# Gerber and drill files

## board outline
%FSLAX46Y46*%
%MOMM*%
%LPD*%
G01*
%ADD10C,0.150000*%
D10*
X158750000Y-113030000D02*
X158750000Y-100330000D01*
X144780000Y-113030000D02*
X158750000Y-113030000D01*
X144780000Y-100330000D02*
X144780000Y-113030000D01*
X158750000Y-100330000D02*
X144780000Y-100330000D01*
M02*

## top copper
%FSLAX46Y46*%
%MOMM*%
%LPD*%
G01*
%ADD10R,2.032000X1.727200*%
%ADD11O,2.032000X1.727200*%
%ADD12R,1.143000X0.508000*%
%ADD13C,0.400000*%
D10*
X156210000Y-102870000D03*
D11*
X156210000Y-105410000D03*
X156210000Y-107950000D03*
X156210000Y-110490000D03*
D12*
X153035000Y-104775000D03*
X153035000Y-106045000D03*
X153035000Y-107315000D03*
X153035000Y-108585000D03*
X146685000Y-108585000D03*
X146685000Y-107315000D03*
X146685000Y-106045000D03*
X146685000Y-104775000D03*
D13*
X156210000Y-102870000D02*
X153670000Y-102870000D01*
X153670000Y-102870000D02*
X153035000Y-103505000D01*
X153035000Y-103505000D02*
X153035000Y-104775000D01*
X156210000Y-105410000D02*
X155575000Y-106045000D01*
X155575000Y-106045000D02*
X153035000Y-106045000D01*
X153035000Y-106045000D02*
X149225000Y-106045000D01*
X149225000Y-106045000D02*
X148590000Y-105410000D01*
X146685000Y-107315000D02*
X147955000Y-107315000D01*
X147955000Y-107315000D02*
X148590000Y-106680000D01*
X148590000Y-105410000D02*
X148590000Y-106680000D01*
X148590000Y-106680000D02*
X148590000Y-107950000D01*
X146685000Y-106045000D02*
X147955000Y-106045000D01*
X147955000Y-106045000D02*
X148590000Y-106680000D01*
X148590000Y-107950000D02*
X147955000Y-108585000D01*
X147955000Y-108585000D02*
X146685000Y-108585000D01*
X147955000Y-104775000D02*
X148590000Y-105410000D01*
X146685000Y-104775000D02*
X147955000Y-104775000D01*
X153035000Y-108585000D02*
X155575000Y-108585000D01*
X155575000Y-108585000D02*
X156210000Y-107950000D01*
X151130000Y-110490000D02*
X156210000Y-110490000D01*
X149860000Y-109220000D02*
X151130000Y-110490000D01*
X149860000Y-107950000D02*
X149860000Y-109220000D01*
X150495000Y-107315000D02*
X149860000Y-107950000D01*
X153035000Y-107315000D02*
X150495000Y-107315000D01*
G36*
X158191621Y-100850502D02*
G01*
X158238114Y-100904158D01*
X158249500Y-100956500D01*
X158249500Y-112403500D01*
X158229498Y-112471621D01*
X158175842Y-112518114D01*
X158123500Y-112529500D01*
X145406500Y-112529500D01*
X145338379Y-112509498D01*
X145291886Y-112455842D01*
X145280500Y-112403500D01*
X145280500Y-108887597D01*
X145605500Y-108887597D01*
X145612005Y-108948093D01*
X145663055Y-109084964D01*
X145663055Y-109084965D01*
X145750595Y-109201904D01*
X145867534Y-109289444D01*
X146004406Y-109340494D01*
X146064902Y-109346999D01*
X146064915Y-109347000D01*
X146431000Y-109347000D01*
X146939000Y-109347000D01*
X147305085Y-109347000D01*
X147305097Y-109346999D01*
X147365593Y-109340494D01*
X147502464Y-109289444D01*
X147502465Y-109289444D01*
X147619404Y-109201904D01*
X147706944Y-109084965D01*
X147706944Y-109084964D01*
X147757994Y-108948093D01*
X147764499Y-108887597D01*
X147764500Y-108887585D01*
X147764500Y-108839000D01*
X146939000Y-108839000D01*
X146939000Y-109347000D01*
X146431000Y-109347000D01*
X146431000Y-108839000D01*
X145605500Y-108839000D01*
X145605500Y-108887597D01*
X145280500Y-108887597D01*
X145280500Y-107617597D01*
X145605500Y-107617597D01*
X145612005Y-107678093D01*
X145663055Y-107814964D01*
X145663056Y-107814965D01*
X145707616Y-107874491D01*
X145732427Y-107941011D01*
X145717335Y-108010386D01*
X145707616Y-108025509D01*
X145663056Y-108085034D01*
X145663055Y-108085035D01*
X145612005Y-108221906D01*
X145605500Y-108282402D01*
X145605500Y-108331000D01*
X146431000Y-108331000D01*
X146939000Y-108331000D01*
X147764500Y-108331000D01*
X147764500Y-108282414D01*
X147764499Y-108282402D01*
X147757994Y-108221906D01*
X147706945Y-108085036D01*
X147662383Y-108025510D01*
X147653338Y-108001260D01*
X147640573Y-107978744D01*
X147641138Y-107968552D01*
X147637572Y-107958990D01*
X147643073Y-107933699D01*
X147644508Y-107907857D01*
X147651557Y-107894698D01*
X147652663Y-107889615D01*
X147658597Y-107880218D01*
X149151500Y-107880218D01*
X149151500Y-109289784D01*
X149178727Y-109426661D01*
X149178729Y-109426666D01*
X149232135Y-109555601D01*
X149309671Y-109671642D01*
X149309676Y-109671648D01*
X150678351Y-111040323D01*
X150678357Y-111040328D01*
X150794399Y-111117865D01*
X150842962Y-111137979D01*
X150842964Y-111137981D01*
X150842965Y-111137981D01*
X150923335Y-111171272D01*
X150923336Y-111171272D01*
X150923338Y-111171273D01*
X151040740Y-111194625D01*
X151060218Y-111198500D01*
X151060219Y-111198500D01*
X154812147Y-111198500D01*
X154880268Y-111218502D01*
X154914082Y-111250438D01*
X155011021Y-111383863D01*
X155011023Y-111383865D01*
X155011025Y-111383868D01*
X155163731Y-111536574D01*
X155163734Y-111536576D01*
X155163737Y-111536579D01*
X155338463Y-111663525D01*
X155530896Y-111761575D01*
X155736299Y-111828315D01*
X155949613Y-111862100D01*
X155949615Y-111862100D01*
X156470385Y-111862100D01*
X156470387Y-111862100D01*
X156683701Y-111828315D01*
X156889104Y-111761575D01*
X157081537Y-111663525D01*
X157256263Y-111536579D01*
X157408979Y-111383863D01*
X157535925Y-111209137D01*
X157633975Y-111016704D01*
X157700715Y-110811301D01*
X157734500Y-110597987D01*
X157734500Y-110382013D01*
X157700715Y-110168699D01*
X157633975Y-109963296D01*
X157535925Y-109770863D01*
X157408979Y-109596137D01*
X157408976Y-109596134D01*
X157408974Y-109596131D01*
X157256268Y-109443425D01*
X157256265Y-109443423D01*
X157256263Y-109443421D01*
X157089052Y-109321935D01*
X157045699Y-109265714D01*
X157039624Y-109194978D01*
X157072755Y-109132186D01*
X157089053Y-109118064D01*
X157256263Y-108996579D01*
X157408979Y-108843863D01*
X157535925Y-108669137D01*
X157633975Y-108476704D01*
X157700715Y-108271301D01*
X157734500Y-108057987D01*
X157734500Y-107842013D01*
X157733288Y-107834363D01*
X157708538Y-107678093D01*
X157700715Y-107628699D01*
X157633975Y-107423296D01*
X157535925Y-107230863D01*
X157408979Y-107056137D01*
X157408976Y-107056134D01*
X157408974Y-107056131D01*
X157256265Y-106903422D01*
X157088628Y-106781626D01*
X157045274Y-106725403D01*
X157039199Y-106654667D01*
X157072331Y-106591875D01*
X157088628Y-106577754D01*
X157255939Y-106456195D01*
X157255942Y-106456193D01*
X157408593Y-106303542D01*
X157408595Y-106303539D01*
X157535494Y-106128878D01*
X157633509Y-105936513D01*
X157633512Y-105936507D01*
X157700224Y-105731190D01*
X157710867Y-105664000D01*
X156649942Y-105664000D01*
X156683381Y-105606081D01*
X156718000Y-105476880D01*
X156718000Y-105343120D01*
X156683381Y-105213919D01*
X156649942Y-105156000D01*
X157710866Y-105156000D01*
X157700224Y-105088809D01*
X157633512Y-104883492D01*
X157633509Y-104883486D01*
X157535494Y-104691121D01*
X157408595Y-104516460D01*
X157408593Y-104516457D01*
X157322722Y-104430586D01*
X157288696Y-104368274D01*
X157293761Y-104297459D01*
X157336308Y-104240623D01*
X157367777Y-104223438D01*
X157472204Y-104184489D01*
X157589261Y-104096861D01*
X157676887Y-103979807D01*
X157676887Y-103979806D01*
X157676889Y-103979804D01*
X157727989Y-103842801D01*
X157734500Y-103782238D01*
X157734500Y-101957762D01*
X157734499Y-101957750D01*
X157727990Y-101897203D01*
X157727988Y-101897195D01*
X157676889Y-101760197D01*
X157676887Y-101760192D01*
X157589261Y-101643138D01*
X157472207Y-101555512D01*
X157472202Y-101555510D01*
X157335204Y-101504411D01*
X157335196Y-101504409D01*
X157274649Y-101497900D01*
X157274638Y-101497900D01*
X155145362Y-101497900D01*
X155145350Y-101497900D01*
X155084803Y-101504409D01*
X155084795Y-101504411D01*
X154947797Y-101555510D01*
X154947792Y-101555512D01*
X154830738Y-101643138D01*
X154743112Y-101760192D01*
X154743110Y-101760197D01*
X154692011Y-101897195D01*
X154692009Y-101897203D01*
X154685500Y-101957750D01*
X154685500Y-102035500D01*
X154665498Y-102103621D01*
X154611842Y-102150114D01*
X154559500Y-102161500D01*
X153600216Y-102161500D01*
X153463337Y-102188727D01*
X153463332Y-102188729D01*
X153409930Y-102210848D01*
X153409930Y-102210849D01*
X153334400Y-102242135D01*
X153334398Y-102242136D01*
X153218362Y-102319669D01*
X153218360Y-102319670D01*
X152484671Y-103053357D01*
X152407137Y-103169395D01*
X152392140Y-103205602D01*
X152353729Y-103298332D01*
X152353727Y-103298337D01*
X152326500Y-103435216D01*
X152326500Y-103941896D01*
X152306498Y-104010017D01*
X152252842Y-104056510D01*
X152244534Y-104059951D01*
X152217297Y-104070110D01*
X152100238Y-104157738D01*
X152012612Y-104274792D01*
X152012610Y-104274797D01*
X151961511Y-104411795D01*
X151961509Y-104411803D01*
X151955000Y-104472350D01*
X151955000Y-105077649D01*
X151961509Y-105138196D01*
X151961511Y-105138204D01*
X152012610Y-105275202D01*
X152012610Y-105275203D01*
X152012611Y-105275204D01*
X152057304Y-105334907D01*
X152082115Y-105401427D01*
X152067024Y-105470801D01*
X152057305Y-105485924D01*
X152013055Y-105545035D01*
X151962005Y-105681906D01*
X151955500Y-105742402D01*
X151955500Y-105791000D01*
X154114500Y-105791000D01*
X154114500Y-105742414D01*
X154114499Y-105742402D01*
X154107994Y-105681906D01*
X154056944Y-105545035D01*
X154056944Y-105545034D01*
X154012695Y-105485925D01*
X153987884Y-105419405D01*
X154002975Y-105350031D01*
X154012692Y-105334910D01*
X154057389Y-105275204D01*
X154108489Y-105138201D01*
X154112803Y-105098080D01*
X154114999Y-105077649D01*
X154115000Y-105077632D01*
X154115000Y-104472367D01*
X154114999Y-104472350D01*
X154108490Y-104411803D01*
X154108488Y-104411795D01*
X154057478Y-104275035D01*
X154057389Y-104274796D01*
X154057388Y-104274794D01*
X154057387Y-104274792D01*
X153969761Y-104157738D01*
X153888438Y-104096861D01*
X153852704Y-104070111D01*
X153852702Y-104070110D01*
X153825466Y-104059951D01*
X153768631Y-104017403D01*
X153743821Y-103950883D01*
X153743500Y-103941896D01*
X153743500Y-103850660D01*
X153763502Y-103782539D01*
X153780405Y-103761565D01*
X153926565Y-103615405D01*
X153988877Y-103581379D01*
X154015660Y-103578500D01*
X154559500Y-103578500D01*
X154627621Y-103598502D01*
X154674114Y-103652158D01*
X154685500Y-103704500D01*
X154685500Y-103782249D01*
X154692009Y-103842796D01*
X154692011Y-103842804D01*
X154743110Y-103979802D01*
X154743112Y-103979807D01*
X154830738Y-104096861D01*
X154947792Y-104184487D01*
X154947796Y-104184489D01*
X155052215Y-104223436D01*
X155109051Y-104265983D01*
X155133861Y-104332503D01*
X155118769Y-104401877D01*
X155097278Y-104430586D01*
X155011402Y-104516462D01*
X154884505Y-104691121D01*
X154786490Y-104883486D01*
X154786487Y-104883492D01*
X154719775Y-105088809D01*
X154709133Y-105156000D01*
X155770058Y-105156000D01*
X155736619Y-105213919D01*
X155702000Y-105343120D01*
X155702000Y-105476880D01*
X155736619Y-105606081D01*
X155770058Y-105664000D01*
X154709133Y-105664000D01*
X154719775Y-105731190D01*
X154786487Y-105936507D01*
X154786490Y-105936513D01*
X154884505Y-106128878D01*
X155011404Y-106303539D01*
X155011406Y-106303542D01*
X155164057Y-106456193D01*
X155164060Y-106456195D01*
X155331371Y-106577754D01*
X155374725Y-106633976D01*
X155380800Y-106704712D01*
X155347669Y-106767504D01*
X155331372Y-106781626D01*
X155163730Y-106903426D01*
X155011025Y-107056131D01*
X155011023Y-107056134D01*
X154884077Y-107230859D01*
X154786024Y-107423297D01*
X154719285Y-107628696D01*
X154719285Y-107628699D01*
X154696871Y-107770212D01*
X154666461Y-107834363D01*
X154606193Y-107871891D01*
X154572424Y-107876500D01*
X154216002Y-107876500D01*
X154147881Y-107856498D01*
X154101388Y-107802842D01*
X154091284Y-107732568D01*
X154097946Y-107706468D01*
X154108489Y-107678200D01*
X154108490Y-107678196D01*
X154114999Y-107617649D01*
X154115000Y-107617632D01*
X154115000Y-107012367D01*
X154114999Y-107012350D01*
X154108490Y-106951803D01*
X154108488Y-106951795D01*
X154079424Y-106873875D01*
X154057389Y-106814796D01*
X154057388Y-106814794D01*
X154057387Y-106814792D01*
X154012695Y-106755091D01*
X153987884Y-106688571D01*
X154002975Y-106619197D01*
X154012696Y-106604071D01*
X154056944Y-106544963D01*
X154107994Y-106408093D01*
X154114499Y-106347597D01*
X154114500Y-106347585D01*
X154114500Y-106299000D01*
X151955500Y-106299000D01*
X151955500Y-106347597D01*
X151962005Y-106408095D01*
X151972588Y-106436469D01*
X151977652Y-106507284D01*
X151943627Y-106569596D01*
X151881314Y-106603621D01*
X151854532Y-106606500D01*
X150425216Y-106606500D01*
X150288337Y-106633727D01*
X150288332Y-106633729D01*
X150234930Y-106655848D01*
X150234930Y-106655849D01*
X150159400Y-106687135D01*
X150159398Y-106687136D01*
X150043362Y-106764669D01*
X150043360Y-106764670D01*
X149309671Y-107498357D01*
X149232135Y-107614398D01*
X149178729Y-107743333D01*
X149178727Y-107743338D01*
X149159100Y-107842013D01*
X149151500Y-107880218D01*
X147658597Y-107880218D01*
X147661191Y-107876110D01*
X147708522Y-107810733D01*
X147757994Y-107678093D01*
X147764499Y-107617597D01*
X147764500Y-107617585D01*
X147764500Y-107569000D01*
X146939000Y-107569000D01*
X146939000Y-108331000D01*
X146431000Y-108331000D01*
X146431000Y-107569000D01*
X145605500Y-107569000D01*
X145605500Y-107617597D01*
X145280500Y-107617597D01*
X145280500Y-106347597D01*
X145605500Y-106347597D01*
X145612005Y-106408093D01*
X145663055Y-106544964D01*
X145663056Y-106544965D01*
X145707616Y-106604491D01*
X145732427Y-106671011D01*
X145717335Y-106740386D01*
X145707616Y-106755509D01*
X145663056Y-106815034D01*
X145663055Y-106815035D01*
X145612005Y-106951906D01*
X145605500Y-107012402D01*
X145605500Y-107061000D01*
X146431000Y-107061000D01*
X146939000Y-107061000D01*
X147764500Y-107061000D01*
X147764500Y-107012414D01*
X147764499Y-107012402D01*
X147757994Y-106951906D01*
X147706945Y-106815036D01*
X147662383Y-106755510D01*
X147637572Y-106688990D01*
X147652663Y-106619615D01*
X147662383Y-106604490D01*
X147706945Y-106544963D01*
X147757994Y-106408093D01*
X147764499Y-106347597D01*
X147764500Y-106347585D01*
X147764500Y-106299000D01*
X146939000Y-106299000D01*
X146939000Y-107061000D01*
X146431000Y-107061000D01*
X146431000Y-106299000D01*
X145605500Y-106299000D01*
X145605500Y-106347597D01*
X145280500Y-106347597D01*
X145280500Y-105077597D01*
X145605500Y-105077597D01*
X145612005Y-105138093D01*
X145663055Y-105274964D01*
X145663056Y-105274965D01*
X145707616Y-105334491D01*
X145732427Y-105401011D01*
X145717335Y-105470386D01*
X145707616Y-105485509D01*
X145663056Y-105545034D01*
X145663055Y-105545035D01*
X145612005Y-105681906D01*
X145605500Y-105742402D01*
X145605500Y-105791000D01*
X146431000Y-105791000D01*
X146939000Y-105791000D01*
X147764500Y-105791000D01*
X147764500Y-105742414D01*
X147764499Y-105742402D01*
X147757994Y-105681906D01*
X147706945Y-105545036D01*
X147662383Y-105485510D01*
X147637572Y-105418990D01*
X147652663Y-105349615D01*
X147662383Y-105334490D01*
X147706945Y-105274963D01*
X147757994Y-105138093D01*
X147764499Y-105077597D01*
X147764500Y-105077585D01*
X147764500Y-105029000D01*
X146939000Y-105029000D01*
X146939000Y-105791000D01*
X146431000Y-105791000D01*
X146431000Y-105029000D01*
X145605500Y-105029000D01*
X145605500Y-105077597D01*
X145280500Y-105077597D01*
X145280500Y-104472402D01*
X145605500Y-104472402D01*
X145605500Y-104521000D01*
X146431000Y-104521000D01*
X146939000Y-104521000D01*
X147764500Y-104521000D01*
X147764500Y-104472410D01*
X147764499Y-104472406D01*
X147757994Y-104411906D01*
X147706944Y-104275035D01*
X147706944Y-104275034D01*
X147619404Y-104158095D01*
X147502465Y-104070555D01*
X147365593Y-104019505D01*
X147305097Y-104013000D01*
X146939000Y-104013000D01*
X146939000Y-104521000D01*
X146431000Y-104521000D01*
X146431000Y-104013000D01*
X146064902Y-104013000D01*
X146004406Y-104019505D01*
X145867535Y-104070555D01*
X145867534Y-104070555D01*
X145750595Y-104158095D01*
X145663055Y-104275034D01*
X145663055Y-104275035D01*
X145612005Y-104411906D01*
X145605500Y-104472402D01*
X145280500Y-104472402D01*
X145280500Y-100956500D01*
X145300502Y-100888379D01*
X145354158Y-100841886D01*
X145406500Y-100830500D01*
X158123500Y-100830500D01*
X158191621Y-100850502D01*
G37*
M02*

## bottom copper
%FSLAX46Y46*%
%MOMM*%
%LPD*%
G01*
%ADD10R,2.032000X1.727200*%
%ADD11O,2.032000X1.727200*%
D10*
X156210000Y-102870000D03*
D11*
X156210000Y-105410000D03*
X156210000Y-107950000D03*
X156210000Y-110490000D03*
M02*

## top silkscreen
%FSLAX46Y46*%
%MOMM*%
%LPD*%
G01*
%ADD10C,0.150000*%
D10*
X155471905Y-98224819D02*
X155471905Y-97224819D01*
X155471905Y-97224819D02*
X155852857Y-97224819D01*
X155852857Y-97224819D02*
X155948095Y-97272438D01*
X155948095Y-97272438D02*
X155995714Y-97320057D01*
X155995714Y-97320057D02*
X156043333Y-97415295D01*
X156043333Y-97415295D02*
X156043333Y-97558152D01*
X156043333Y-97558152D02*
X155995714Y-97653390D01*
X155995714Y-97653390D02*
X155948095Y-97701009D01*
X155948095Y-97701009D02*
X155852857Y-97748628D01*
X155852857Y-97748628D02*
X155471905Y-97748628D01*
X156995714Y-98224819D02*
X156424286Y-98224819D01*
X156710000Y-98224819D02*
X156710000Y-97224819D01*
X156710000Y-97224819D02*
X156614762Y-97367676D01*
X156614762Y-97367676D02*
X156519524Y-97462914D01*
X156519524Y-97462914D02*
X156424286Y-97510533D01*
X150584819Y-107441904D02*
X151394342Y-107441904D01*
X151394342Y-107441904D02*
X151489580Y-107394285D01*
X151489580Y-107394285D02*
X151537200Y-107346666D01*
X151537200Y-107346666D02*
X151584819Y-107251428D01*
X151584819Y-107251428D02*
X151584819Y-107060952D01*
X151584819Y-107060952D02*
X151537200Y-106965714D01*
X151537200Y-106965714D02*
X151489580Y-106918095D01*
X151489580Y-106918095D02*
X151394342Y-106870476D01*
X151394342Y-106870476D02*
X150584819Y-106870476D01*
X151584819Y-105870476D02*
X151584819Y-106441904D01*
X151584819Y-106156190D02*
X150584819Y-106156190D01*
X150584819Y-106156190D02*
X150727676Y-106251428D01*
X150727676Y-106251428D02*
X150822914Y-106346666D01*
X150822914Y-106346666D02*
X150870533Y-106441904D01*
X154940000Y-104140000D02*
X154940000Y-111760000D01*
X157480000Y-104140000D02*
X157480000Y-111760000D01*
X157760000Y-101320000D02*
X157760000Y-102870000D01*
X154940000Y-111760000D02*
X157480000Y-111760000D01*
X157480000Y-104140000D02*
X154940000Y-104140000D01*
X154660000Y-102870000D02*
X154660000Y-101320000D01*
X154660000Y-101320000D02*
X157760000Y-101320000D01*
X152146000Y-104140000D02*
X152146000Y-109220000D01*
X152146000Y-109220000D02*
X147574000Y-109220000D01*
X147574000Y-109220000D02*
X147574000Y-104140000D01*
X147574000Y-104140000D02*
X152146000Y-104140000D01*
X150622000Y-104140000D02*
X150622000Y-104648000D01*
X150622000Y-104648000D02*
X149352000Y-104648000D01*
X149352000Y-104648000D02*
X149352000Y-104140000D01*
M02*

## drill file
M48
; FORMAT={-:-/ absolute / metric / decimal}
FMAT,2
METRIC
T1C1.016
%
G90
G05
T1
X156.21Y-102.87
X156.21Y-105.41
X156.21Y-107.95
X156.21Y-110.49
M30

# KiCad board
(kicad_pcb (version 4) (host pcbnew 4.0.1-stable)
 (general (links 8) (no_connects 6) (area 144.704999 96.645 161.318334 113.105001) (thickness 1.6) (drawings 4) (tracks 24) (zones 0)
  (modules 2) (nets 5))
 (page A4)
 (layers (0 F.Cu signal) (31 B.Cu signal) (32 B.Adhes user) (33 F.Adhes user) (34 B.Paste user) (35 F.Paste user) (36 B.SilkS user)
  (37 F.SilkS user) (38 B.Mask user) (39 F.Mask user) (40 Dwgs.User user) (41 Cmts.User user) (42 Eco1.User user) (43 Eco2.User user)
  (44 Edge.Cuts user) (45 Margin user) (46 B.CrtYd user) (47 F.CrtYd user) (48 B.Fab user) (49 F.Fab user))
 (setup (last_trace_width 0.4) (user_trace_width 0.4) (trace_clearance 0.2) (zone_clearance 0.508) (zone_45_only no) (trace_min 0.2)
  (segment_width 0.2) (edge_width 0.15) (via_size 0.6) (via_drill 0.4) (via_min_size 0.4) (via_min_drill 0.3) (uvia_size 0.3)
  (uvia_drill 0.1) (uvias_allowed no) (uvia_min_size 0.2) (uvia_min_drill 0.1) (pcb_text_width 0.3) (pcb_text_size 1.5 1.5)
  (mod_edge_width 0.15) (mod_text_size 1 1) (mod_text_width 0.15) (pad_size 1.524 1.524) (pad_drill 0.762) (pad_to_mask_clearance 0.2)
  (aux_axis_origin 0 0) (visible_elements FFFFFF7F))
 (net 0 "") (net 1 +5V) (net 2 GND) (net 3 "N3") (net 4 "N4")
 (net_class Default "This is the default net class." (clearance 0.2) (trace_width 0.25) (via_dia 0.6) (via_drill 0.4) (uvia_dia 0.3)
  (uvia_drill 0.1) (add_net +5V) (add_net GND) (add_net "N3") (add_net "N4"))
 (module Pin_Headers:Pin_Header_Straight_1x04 (layer F.Cu) (at 156.21 102.87)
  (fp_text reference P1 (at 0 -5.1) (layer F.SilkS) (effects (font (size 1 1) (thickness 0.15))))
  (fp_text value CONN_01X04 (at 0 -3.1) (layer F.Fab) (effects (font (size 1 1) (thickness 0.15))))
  (fp_line (start -1.27 1.27) (end -1.27 8.89) (layer F.SilkS) (width 0.15))
  (fp_line (start 1.27 1.27) (end 1.27 8.89) (layer F.SilkS) (width 0.15))
  (fp_line (start 1.55 -1.55) (end 1.55 0) (layer F.SilkS) (width 0.15))
  (fp_line (start -1.27 8.89) (end 1.27 8.89) (layer F.SilkS) (width 0.15))
  (fp_line (start 1.27 1.27) (end -1.27 1.27) (layer F.SilkS) (width 0.15))
  (fp_line (start -1.55 0) (end -1.55 -1.55) (layer F.SilkS) (width 0.15))
  (fp_line (start -1.55 -1.55) (end 1.55 -1.55) (layer F.SilkS) (width 0.15))
  (pad 1 thru_hole rect (at 0 0) (size 2.032 1.7272) (drill 1.016) (layers *.Cu *.Mask) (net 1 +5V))
  (pad 2 thru_hole oval (at 0 2.54) (size 2.032 1.7272) (drill 1.016) (layers *.Cu *.Mask) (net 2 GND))
  (pad 3 thru_hole oval (at 0 5.08) (size 2.032 1.7272) (drill 1.016) (layers *.Cu *.Mask) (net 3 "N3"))
  (pad 4 thru_hole oval (at 0 7.62) (size 2.032 1.7272) (drill 1.016) (layers *.Cu *.Mask) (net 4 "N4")))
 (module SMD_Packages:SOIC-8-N (layer F.Cu) (at 149.86 106.68 270)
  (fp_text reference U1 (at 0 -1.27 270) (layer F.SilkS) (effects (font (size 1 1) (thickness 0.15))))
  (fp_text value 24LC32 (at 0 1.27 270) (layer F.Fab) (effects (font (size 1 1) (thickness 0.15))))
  (fp_line (start -2.54 -2.286) (end 2.54 -2.286) (layer F.SilkS) (width 0.15))
  (fp_line (start 2.54 -2.286) (end 2.54 2.286) (layer F.SilkS) (width 0.15))
  (fp_line (start 2.54 2.286) (end -2.54 2.286) (layer F.SilkS) (width 0.15))
  (fp_line (start -2.54 2.286) (end -2.54 -2.286) (layer F.SilkS) (width 0.15))
  (fp_line (start -2.54 -0.762) (end -2.032 -0.762) (layer F.SilkS) (width 0.15))
  (fp_line (start -2.032 -0.762) (end -2.032 0.508) (layer F.SilkS) (width 0.15))
  (fp_line (start -2.032 0.508) (end -2.54 0.508) (layer F.SilkS) (width 0.15))
  (pad 8 smd rect (at -1.905 -3.175 270) (size 0.508 1.143) (layers F.Cu F.Paste F.Mask) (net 1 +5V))
  (pad 7 smd rect (at -0.635 -3.175 270) (size 0.508 1.143) (layers F.Cu F.Paste F.Mask) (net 2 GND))
  (pad 6 smd rect (at 0.635 -3.175 270) (size 0.508 1.143) (layers F.Cu F.Paste F.Mask) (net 4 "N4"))
  (pad 5 smd rect (at 1.905 -3.175 270) (size 0.508 1.143) (layers F.Cu F.Paste F.Mask) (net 3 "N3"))
  (pad 4 smd rect (at 1.905 3.175 270) (size 0.508 1.143) (layers F.Cu F.Paste F.Mask) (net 2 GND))
  (pad 3 smd rect (at 0.635 3.175 270) (size 0.508 1.143) (layers F.Cu F.Paste F.Mask) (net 2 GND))
  (pad 2 smd rect (at -0.635 3.175 270) (size 0.508 1.143) (layers F.Cu F.Paste F.Mask) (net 2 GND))
  (pad 1 smd rect (at -1.905 3.175 270) (size 0.508 1.143) (layers F.Cu F.Paste F.Mask) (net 2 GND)))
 (gr_line (start 158.75 113.03) (end 158.75 100.33) (layer Edge.Cuts) (width 0.15))
 (gr_line (start 144.78 113.03) (end 158.75 113.03) (layer Edge.Cuts) (width 0.15))
 (gr_line (start 144.78 100.33) (end 144.78 113.03) (layer Edge.Cuts) (width 0.15))
 (gr_line (start 158.75 100.33) (end 144.78 100.33) (layer Edge.Cuts) (width 0.15))
 (segment (start 156.21 102.87) (end 153.67 102.87) (width 0.4) (layer F.Cu) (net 1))
 (segment (start 153.67 102.87) (end 153.035 103.505) (width 0.4) (layer F.Cu) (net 1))
 (segment (start 153.035 103.505) (end 153.035 104.775) (width 0.4) (layer F.Cu) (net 1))
 (segment (start 156.21 105.41) (end 155.575 106.045) (width 0.4) (layer F.Cu) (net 2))
 (segment (start 155.575 106.045) (end 153.035 106.045) (width 0.4) (layer F.Cu) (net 2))
 (segment (start 153.035 106.045) (end 149.225 106.045) (width 0.4) (layer F.Cu) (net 2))
 (segment (start 149.225 106.045) (end 148.59 105.41) (width 0.4) (layer F.Cu) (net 2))
 (segment (start 146.685 107.315) (end 147.955 107.315) (width 0.4) (layer F.Cu) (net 2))
 (segment (start 147.955 107.315) (end 148.59 106.68) (width 0.4) (layer F.Cu) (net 2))
 (segment (start 148.59 105.41) (end 148.59 106.68) (width 0.4) (layer F.Cu) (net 2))
 (segment (start 148.59 106.68) (end 148.59 107.95) (width 0.4) (layer F.Cu) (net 2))
 (segment (start 146.685 106.045) (end 147.955 106.045) (width 0.4) (layer F.Cu) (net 2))
 (segment (start 147.955 106.045) (end 148.59 106.68) (width 0.4) (layer F.Cu) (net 2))
 (segment (start 148.59 107.95) (end 147.955 108.585) (width 0.4) (layer F.Cu) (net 2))
 (segment (start 147.955 108.585) (end 146.685 108.585) (width 0.4) (layer F.Cu) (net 2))
 (segment (start 147.955 104.775) (end 148.59 105.41) (width 0.4) (layer F.Cu) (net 2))
 (segment (start 146.685 104.775) (end 147.955 104.775) (width 0.4) (layer F.Cu) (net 2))
 (segment (start 153.035 108.585) (end 155.575 108.585) (width 0.4) (layer F.Cu) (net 3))
 (segment (start 155.575 108.585) (end 156.21 107.95) (width 0.4) (layer F.Cu) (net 3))
 (segment (start 151.13 110.49) (end 156.21 110.49) (width 0.4) (layer F.Cu) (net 4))
 (segment (start 149.86 109.22) (end 151.13 110.49) (width 0.4) (layer F.Cu) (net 4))
 (segment (start 149.86 107.95) (end 149.86 109.22) (width 0.4) (layer F.Cu) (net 4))
 (segment (start 150.495 107.315) (end 149.86 107.95) (width 0.4) (layer F.Cu) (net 4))
 (segment (start 153.035 107.315) (end 150.495 107.315) (width 0.4) (layer F.Cu) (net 4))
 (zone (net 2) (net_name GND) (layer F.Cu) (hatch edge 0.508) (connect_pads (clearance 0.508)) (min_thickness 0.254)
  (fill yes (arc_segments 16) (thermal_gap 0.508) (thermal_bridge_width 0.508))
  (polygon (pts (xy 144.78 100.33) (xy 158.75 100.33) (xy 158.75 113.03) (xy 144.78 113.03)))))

